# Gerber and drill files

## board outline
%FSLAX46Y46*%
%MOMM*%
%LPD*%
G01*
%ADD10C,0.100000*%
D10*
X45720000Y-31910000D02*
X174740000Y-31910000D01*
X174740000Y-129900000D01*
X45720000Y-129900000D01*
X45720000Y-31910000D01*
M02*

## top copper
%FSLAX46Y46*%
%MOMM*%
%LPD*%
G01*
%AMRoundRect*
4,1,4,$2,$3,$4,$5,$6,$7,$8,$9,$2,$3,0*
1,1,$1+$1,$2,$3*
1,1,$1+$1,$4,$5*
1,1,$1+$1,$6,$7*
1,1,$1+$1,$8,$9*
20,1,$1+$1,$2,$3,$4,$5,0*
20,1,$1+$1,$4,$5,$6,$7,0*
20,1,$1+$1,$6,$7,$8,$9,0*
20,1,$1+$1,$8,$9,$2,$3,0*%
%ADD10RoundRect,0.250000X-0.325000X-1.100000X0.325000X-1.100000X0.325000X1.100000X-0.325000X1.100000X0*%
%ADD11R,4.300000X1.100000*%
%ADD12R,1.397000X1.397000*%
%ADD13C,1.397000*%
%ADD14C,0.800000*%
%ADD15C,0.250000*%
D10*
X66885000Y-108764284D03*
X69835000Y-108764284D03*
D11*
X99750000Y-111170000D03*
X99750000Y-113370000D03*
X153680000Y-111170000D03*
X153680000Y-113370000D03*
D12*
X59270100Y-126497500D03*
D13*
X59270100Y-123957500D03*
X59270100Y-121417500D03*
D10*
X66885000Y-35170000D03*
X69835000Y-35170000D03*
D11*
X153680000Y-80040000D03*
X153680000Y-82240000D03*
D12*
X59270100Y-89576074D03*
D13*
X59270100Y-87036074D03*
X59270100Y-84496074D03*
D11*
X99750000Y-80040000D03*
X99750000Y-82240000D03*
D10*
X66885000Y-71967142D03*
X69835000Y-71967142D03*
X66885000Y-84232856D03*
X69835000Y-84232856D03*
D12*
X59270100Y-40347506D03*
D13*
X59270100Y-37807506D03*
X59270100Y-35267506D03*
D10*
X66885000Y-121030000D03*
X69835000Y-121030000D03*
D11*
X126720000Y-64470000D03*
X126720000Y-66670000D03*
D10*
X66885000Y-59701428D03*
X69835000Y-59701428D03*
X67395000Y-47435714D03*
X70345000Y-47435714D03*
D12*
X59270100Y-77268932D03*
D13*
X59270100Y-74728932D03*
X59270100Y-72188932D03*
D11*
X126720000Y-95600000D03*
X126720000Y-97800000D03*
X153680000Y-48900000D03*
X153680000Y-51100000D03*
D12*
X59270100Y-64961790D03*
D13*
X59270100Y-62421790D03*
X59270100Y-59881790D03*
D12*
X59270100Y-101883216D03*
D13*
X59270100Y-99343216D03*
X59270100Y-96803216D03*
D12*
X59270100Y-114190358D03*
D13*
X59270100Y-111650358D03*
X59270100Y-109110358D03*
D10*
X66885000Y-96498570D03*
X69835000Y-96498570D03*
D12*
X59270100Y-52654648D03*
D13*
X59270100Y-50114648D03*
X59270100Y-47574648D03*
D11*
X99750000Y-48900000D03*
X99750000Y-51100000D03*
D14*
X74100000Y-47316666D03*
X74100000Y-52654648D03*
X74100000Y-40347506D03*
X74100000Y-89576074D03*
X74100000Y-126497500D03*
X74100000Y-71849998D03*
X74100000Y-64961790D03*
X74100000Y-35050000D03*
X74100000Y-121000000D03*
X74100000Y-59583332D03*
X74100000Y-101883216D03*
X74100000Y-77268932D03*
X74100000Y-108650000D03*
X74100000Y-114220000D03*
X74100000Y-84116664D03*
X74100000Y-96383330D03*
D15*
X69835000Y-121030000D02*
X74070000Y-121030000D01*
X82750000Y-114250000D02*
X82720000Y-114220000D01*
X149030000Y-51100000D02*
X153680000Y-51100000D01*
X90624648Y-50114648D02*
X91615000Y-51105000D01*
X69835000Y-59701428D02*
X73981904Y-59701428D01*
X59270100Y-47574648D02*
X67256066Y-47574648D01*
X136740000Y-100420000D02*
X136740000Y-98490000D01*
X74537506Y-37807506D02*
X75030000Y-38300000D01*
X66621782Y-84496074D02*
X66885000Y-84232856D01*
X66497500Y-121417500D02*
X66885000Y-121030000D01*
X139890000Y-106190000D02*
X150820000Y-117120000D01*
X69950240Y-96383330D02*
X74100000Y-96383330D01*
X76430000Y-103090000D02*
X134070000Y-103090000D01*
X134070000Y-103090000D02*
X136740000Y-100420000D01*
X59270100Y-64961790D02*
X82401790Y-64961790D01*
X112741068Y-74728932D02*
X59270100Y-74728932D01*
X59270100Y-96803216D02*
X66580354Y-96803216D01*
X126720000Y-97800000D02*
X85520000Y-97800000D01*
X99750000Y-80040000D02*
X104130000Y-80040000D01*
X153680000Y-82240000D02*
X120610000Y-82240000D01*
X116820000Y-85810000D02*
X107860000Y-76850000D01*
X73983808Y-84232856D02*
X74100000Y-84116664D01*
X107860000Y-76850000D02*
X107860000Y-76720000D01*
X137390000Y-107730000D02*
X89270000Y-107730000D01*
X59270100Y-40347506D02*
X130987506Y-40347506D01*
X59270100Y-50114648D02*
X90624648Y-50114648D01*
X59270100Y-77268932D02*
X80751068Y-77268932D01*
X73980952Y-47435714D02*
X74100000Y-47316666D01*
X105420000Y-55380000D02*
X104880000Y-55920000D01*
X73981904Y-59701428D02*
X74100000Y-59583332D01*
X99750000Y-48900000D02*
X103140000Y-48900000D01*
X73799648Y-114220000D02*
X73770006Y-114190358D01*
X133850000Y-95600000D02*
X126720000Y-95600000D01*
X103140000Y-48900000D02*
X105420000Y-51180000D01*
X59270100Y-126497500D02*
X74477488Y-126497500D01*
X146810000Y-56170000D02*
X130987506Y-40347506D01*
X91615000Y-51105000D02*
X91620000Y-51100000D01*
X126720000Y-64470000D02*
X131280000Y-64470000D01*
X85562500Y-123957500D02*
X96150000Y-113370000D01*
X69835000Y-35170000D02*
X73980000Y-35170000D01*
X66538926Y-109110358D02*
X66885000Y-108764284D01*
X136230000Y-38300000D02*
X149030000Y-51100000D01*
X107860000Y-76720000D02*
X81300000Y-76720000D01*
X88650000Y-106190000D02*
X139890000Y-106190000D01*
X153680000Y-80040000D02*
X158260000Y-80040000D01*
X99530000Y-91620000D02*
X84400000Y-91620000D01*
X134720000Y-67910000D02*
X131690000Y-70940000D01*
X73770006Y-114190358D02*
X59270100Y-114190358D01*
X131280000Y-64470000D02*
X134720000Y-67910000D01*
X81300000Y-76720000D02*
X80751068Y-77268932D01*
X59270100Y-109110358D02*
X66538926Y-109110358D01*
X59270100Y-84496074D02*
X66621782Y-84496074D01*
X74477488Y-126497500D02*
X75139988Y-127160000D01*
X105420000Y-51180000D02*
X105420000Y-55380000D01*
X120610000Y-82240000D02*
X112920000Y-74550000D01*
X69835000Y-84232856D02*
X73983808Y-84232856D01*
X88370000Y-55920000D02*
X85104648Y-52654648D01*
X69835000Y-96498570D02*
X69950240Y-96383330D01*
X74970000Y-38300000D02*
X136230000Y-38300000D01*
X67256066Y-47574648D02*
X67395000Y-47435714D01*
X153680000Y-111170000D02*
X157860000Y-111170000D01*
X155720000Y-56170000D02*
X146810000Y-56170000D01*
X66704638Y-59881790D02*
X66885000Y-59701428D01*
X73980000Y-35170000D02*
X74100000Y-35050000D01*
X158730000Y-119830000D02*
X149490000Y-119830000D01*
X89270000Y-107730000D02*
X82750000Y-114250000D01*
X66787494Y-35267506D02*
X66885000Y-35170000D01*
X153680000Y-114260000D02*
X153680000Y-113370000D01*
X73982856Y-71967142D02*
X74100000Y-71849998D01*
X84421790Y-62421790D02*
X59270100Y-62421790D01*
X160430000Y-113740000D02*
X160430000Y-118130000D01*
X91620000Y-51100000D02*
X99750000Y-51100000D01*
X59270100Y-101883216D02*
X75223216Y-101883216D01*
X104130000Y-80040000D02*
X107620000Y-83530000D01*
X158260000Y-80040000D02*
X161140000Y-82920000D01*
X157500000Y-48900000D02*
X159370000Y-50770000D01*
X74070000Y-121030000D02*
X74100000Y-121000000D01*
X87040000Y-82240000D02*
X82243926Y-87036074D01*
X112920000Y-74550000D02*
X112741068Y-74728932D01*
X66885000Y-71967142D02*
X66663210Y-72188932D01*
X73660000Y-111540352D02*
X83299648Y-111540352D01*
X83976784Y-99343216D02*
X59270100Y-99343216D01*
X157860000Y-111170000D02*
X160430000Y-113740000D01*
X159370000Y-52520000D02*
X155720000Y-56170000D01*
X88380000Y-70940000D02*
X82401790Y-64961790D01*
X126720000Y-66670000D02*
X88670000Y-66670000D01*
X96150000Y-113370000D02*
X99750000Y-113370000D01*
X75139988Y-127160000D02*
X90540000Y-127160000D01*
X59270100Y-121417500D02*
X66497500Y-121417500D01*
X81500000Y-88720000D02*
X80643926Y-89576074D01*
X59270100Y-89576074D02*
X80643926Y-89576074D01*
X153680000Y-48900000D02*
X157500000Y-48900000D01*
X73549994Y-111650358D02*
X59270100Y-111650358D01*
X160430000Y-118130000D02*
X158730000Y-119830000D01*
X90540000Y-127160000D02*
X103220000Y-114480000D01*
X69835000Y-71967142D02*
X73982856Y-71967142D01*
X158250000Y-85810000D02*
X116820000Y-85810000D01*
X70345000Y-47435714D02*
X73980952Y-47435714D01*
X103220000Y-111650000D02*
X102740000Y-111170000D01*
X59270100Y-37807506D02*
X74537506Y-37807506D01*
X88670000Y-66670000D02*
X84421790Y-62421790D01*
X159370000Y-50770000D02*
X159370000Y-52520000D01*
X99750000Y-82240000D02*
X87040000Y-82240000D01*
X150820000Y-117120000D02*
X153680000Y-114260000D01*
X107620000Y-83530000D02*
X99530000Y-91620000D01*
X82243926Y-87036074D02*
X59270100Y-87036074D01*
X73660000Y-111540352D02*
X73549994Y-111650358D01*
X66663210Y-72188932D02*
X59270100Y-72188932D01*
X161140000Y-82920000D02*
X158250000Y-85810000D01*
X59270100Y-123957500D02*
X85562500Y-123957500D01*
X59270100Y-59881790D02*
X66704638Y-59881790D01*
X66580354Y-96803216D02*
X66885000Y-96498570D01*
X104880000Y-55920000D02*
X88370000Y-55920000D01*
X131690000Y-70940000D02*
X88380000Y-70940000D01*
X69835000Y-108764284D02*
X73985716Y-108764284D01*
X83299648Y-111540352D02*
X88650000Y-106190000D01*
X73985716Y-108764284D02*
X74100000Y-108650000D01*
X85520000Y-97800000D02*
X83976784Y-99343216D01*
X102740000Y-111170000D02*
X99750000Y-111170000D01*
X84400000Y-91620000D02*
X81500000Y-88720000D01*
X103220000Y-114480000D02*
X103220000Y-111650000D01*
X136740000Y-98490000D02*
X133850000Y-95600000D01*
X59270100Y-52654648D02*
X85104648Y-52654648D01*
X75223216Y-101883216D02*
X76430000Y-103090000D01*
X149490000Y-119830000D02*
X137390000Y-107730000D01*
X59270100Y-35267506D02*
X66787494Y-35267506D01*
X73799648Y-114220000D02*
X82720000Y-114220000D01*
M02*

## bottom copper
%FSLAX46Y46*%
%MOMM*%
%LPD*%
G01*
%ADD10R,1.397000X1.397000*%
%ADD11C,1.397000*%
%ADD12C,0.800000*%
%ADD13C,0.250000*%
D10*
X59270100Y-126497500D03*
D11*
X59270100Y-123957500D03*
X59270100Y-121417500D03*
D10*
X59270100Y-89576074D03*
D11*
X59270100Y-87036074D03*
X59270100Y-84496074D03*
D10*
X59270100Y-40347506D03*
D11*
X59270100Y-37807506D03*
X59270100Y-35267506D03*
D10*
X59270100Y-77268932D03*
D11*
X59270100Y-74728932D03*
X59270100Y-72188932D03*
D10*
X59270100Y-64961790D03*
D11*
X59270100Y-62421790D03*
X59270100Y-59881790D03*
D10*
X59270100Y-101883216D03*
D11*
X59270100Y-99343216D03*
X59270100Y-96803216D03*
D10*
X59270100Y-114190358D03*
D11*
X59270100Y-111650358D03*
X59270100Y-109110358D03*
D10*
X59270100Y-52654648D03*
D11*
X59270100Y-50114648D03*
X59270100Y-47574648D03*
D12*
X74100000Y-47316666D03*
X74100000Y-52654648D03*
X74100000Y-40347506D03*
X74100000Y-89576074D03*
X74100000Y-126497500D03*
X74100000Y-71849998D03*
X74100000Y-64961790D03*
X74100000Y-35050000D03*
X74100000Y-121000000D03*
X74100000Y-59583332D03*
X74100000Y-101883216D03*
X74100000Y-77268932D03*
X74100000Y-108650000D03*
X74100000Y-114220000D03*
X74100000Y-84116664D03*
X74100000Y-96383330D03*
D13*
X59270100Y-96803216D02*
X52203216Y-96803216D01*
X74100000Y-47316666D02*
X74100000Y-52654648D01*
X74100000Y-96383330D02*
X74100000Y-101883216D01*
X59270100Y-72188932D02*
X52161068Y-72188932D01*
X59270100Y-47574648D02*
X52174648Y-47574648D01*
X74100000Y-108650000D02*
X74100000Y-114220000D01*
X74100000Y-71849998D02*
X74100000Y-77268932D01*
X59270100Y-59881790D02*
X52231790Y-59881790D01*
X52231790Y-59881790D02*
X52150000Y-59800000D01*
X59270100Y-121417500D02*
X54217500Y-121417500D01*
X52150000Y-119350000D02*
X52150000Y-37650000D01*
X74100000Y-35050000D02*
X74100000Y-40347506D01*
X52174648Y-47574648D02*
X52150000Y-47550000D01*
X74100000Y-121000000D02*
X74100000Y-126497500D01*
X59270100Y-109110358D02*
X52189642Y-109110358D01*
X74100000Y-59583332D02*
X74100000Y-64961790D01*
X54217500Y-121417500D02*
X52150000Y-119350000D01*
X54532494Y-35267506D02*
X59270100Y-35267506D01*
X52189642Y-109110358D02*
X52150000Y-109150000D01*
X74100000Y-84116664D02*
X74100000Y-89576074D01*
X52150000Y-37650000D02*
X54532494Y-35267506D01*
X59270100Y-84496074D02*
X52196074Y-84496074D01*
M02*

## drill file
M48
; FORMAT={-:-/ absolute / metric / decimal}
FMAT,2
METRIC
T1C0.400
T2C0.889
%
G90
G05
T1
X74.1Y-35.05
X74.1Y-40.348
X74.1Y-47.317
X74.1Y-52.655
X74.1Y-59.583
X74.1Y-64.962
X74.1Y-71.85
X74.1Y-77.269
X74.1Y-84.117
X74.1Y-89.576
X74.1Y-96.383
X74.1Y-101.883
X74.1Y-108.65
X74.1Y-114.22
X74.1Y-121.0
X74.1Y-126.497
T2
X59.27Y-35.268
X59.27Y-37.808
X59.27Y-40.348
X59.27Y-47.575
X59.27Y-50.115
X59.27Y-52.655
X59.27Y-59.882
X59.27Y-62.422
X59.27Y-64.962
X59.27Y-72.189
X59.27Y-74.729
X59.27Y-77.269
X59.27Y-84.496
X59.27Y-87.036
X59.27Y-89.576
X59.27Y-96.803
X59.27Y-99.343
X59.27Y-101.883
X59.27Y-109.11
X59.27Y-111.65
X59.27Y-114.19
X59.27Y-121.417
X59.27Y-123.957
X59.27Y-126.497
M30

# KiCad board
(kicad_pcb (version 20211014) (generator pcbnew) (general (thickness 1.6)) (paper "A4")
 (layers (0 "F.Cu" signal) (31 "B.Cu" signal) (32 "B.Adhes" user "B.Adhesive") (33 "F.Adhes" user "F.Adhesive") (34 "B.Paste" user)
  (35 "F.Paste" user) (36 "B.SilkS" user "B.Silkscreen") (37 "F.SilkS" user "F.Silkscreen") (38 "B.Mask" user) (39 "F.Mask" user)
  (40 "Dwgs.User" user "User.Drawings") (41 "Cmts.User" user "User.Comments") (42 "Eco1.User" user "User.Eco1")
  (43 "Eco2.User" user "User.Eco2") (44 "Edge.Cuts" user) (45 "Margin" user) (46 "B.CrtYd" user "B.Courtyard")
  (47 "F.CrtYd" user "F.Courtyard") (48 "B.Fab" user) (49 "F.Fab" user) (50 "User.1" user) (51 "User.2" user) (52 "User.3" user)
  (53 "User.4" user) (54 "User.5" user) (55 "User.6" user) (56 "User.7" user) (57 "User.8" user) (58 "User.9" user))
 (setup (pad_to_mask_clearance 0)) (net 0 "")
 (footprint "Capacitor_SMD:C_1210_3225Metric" (layer "F.Cu") (at 68.36 108.764284)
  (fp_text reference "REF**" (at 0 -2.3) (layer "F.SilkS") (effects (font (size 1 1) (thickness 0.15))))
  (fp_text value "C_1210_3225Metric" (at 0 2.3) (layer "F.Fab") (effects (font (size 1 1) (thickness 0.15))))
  (pad "1" smd roundrect (at -1.475 0) (size 1.15 2.7) (layers "F.Cu" "F.Paste" "F.Mask") (roundrect_rratio 0.2173913043))
  (pad "2" smd roundrect (at 1.475 0) (size 1.15 2.7) (layers "F.Cu" "F.Paste" "F.Mask") (roundrect_rratio 0.2173913043)))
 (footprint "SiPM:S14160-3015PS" (layer "F.Cu") (at 100 112.27)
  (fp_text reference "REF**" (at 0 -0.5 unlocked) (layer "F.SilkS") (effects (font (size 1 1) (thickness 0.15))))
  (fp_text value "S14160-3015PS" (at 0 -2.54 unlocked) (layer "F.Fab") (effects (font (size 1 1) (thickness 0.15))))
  (pad "1" smd rect (at -0.25 -1.1) (size 4.3 1.1) (layers "F.Cu" "F.Paste" "F.Mask"))
  (pad "2" smd rect (at -0.25 1.1) (size 4.3 1.1) (layers "F.Cu" "F.Paste" "F.Mask")))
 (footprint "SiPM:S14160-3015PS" (layer "F.Cu") (at 153.93 112.27)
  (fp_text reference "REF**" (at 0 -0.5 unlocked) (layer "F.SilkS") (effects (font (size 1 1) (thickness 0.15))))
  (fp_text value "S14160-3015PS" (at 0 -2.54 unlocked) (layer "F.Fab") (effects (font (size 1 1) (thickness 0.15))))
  (pad "1" smd rect (at -0.25 -1.1) (size 4.3 1.1) (layers "F.Cu" "F.Paste" "F.Mask"))
  (pad "2" smd rect (at -0.25 1.1) (size 4.3 1.1) (layers "F.Cu" "F.Paste" "F.Mask")))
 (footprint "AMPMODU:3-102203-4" (layer "F.Cu") (at 59.2701 126.4975 90)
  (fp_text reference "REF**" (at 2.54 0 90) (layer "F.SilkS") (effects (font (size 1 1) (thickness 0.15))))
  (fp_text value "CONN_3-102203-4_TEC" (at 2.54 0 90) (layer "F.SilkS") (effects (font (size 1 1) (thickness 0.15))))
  (pad "1" thru_hole rect locked (at 0 0 90) (size 1.397 1.397) (drill 0.889) (layers *.Cu *.Mask))
  (pad "2" thru_hole circle locked (at 2.54 0 90) (size 1.397 1.397) (drill 0.889) (layers *.Cu *.Mask))
  (pad "3" thru_hole circle locked (at 5.08 0 90) (size 1.397 1.397) (drill 0.889) (layers *.Cu *.Mask)))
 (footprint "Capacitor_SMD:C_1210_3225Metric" (layer "F.Cu") (at 68.36 35.17)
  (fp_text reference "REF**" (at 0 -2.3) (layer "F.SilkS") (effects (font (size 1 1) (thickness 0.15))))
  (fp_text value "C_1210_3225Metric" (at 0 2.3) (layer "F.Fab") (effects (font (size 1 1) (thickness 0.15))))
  (pad "1" smd roundrect (at -1.475 0) (size 1.15 2.7) (layers "F.Cu" "F.Paste" "F.Mask") (roundrect_rratio 0.2173913043))
  (pad "2" smd roundrect (at 1.475 0) (size 1.15 2.7) (layers "F.Cu" "F.Paste" "F.Mask") (roundrect_rratio 0.2173913043)))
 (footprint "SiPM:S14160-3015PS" (layer "F.Cu") (at 153.93 81.14)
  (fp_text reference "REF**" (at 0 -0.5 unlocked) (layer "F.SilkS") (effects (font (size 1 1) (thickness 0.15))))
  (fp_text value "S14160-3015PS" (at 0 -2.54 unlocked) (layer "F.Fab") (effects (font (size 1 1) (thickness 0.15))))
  (pad "1" smd rect (at -0.25 -1.1) (size 4.3 1.1) (layers "F.Cu" "F.Paste" "F.Mask"))
  (pad "2" smd rect (at -0.25 1.1) (size 4.3 1.1) (layers "F.Cu" "F.Paste" "F.Mask")))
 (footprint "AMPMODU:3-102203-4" (layer "F.Cu") (at 59.2701 89.576074 90)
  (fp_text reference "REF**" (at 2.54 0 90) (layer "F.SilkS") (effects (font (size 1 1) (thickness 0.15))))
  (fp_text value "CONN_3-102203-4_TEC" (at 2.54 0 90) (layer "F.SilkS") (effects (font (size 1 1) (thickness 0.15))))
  (pad "1" thru_hole rect locked (at 0 0 90) (size 1.397 1.397) (drill 0.889) (layers *.Cu *.Mask))
  (pad "2" thru_hole circle locked (at 2.54 0 90) (size 1.397 1.397) (drill 0.889) (layers *.Cu *.Mask))
  (pad "3" thru_hole circle locked (at 5.08 0 90) (size 1.397 1.397) (drill 0.889) (layers *.Cu *.Mask)))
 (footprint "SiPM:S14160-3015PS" (layer "F.Cu") (at 100 81.14)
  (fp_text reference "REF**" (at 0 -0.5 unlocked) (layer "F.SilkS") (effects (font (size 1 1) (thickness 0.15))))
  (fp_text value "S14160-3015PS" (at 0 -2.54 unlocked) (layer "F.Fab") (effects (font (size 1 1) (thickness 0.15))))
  (pad "1" smd rect (at -0.25 -1.1) (size 4.3 1.1) (layers "F.Cu" "F.Paste" "F.Mask"))
  (pad "2" smd rect (at -0.25 1.1) (size 4.3 1.1) (layers "F.Cu" "F.Paste" "F.Mask")))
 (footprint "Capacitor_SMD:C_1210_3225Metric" (layer "F.Cu") (at 68.36 71.967142)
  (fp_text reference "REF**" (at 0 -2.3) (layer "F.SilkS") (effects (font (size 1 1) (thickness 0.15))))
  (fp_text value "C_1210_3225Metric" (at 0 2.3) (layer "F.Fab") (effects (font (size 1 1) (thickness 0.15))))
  (pad "1" smd roundrect (at -1.475 0) (size 1.15 2.7) (layers "F.Cu" "F.Paste" "F.Mask") (roundrect_rratio 0.2173913043))
  (pad "2" smd roundrect (at 1.475 0) (size 1.15 2.7) (layers "F.Cu" "F.Paste" "F.Mask") (roundrect_rratio 0.2173913043)))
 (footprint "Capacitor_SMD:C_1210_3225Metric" (layer "F.Cu") (at 68.36 84.232856)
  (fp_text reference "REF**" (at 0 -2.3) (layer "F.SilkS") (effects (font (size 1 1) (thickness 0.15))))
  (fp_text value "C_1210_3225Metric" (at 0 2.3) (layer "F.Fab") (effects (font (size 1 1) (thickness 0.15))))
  (pad "1" smd roundrect (at -1.475 0) (size 1.15 2.7) (layers "F.Cu" "F.Paste" "F.Mask") (roundrect_rratio 0.2173913043))
  (pad "2" smd roundrect (at 1.475 0) (size 1.15 2.7) (layers "F.Cu" "F.Paste" "F.Mask") (roundrect_rratio 0.2173913043)))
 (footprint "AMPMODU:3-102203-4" (layer "F.Cu") (at 59.2701 40.347506 90)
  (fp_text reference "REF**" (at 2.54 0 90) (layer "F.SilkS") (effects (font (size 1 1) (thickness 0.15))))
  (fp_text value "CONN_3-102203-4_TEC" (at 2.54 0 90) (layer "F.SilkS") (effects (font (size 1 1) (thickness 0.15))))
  (pad "1" thru_hole rect locked (at 0 0 90) (size 1.397 1.397) (drill 0.889) (layers *.Cu *.Mask))
  (pad "2" thru_hole circle locked (at 2.54 0 90) (size 1.397 1.397) (drill 0.889) (layers *.Cu *.Mask))
  (pad "3" thru_hole circle locked (at 5.08 0 90) (size 1.397 1.397) (drill 0.889) (layers *.Cu *.Mask)))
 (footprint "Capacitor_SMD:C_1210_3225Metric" (layer "F.Cu") (at 68.36 121.03)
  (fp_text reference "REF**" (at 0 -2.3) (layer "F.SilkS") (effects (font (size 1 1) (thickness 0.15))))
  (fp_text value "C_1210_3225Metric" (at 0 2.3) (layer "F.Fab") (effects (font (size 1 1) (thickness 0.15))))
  (pad "1" smd roundrect (at -1.475 0) (size 1.15 2.7) (layers "F.Cu" "F.Paste" "F.Mask") (roundrect_rratio 0.2173913043))
  (pad "2" smd roundrect (at 1.475 0) (size 1.15 2.7) (layers "F.Cu" "F.Paste" "F.Mask") (roundrect_rratio 0.2173913043)))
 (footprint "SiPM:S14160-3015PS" (layer "F.Cu") (at 126.97 65.57)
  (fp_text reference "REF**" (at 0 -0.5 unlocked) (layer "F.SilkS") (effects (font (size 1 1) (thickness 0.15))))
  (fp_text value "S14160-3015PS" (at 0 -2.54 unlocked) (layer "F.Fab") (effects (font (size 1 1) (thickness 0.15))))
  (pad "1" smd rect (at -0.25 -1.1) (size 4.3 1.1) (layers "F.Cu" "F.Paste" "F.Mask"))
  (pad "2" smd rect (at -0.25 1.1) (size 4.3 1.1) (layers "F.Cu" "F.Paste" "F.Mask")))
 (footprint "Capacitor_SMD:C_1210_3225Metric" (layer "F.Cu") (at 68.36 59.701428)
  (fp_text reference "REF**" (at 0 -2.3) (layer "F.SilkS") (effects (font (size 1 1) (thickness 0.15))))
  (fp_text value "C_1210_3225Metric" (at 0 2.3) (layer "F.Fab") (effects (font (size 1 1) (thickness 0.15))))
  (pad "1" smd roundrect (at -1.475 0) (size 1.15 2.7) (layers "F.Cu" "F.Paste" "F.Mask") (roundrect_rratio 0.2173913043))
  (pad "2" smd roundrect (at 1.475 0) (size 1.15 2.7) (layers "F.Cu" "F.Paste" "F.Mask") (roundrect_rratio 0.2173913043)))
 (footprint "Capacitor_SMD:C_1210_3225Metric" (layer "F.Cu") (at 68.87 47.435714)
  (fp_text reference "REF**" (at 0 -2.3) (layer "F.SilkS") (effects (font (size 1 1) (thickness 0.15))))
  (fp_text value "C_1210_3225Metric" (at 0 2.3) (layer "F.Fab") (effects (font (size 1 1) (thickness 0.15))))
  (pad "1" smd roundrect (at -1.475 0) (size 1.15 2.7) (layers "F.Cu" "F.Paste" "F.Mask") (roundrect_rratio 0.2173913043))
  (pad "2" smd roundrect (at 1.475 0) (size 1.15 2.7) (layers "F.Cu" "F.Paste" "F.Mask") (roundrect_rratio 0.2173913043)))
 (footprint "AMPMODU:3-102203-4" (layer "F.Cu") (at 59.2701 77.268932 90)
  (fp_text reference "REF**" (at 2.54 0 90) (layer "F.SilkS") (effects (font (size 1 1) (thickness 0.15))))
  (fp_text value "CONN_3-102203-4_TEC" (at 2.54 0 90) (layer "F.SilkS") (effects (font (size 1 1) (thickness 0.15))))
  (pad "1" thru_hole rect locked (at 0 0 90) (size 1.397 1.397) (drill 0.889) (layers *.Cu *.Mask))
  (pad "2" thru_hole circle locked (at 2.54 0 90) (size 1.397 1.397) (drill 0.889) (layers *.Cu *.Mask))
  (pad "3" thru_hole circle locked (at 5.08 0 90) (size 1.397 1.397) (drill 0.889) (layers *.Cu *.Mask)))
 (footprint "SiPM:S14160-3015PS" (layer "F.Cu") (at 126.97 96.7)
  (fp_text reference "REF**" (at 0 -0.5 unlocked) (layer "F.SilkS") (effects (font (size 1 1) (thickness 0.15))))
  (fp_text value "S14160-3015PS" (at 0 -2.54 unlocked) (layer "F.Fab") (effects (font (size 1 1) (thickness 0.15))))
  (pad "1" smd rect (at -0.25 -1.1) (size 4.3 1.1) (layers "F.Cu" "F.Paste" "F.Mask"))
  (pad "2" smd rect (at -0.25 1.1) (size 4.3 1.1) (layers "F.Cu" "F.Paste" "F.Mask")))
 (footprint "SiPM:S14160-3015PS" (layer "F.Cu") (at 153.93 50)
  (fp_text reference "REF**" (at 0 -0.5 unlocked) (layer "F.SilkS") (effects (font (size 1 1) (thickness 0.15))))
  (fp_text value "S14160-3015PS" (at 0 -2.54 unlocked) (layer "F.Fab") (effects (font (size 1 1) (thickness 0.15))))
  (pad "1" smd rect (at -0.25 -1.1) (size 4.3 1.1) (layers "F.Cu" "F.Paste" "F.Mask"))
  (pad "2" smd rect (at -0.25 1.1) (size 4.3 1.1) (layers "F.Cu" "F.Paste" "F.Mask")))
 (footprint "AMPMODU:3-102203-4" (layer "F.Cu") (at 59.2701 64.96179 90)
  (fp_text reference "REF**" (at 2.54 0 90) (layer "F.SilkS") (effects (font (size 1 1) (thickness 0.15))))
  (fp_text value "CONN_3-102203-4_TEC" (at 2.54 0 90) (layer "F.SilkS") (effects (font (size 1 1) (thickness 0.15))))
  (pad "1" thru_hole rect locked (at 0 0 90) (size 1.397 1.397) (drill 0.889) (layers *.Cu *.Mask))
  (pad "2" thru_hole circle locked (at 2.54 0 90) (size 1.397 1.397) (drill 0.889) (layers *.Cu *.Mask))
  (pad "3" thru_hole circle locked (at 5.08 0 90) (size 1.397 1.397) (drill 0.889) (layers *.Cu *.Mask)))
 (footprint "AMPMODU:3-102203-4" (layer "F.Cu") (at 59.2701 101.883216 90)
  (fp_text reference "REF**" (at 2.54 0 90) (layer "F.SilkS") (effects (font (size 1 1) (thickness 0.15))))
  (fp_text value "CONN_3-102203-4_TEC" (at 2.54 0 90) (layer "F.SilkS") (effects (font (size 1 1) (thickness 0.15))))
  (pad "1" thru_hole rect locked (at 0 0 90) (size 1.397 1.397) (drill 0.889) (layers *.Cu *.Mask))
  (pad "2" thru_hole circle locked (at 2.54 0 90) (size 1.397 1.397) (drill 0.889) (layers *.Cu *.Mask))
  (pad "3" thru_hole circle locked (at 5.08 0 90) (size 1.397 1.397) (drill 0.889) (layers *.Cu *.Mask)))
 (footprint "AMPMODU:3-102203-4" (layer "F.Cu") (at 59.2701 114.190358 90)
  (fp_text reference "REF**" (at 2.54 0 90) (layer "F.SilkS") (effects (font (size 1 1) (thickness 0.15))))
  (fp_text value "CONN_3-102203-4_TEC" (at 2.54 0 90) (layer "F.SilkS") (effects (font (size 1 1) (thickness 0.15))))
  (pad "1" thru_hole rect locked (at 0 0 90) (size 1.397 1.397) (drill 0.889) (layers *.Cu *.Mask))
  (pad "2" thru_hole circle locked (at 2.54 0 90) (size 1.397 1.397) (drill 0.889) (layers *.Cu *.Mask))
  (pad "3" thru_hole circle locked (at 5.08 0 90) (size 1.397 1.397) (drill 0.889) (layers *.Cu *.Mask)))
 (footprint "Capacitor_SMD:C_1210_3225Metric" (layer "F.Cu") (at 68.36 96.49857)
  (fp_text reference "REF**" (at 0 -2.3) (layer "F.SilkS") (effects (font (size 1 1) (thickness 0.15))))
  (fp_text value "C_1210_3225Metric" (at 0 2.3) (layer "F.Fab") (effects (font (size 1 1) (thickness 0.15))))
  (pad "1" smd roundrect (at -1.475 0) (size 1.15 2.7) (layers "F.Cu" "F.Paste" "F.Mask") (roundrect_rratio 0.2173913043))
  (pad "2" smd roundrect (at 1.475 0) (size 1.15 2.7) (layers "F.Cu" "F.Paste" "F.Mask") (roundrect_rratio 0.2173913043)))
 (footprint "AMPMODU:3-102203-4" (layer "F.Cu") (at 59.2701 52.654648 90)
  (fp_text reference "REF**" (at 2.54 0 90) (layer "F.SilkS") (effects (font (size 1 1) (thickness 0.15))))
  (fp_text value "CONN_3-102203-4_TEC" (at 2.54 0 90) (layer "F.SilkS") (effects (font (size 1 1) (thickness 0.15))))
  (pad "1" thru_hole rect locked (at 0 0 90) (size 1.397 1.397) (drill 0.889) (layers *.Cu *.Mask))
  (pad "2" thru_hole circle locked (at 2.54 0 90) (size 1.397 1.397) (drill 0.889) (layers *.Cu *.Mask))
  (pad "3" thru_hole circle locked (at 5.08 0 90) (size 1.397 1.397) (drill 0.889) (layers *.Cu *.Mask)))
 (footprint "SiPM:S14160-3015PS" (layer "F.Cu") (at 100 50)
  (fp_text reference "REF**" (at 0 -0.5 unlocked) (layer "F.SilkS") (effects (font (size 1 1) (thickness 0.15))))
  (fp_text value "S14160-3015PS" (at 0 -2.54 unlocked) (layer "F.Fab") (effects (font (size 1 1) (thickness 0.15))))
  (pad "1" smd rect (at -0.25 -1.1) (size 4.3 1.1) (layers "F.Cu" "F.Paste" "F.Mask"))
  (pad "2" smd rect (at -0.25 1.1) (size 4.3 1.1) (layers "F.Cu" "F.Paste" "F.Mask")))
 (gr_rect (start 45.72 31.91) (end 174.74 129.9) (layer "Edge.Cuts") (width 0.1) (fill none))
 (segment (start 69.835 121.03) (end 74.07 121.03) (width 0.25) (layer "F.Cu") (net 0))
 (segment (start 82.75 114.25) (end 82.72 114.22) (width 0.25) (layer "F.Cu") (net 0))
 (segment (start 149.03 51.1) (end 153.68 51.1) (width 0.25) (layer "F.Cu") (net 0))
 (segment (start 90.624648 50.114648) (end 91.615 51.105) (width 0.25) (layer "F.Cu") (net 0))
 (segment (start 69.835 59.701428) (end 73.981904 59.701428) (width 0.25) (layer "F.Cu") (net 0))
 (segment (start 59.2701 47.574648) (end 67.256066 47.574648) (width 0.25) (layer "F.Cu") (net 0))
 (segment (start 136.74 100.42) (end 136.74 98.49) (width 0.25) (layer "F.Cu") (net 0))
 (segment (start 74.537506 37.807506) (end 75.03 38.3) (width 0.25) (layer "F.Cu") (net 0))
 (segment (start 66.621782 84.496074) (end 66.885 84.232856) (width 0.25) (layer "F.Cu") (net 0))
 (segment (start 66.4975 121.4175) (end 66.885 121.03) (width 0.25) (layer "F.Cu") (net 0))
 (segment (start 139.89 106.19) (end 150.82 117.12) (width 0.25) (layer "F.Cu") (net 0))
 (segment (start 69.95024 96.38333) (end 74.1 96.38333) (width 0.25) (layer "F.Cu") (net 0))
 (segment (start 76.43 103.09) (end 134.07 103.09) (width 0.25) (layer "F.Cu") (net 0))
 (segment (start 134.07 103.09) (end 136.74 100.42) (width 0.25) (layer "F.Cu") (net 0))
 (segment (start 59.2701 64.96179) (end 82.40179 64.96179) (width 0.25) (layer "F.Cu") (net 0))
 (segment (start 112.741068 74.728932) (end 59.2701 74.728932) (width 0.25) (layer "F.Cu") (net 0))
 (segment (start 59.2701 96.803216) (end 66.580354 96.803216) (width 0.25) (layer "F.Cu") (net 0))
 (segment (start 126.72 97.8) (end 85.52 97.8) (width 0.25) (layer "F.Cu") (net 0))
 (segment (start 99.75 80.04) (end 104.13 80.04) (width 0.25) (layer "F.Cu") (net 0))
 (segment (start 153.68 82.24) (end 120.61 82.24) (width 0.25) (layer "F.Cu") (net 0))
 (segment (start 116.82 85.81) (end 107.86 76.85) (width 0.25) (layer "F.Cu") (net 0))
 (segment (start 73.983808 84.232856) (end 74.1 84.116664) (width 0.25) (layer "F.Cu") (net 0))
 (segment (start 107.86 76.85) (end 107.86 76.72) (width 0.25) (layer "F.Cu") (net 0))
 (segment (start 137.39 107.73) (end 89.27 107.73) (width 0.25) (layer "F.Cu") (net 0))
 (segment (start 59.2701 40.347506) (end 130.987506 40.347506) (width 0.25) (layer "F.Cu") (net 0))
 (segment (start 59.2701 50.114648) (end 90.624648 50.114648) (width 0.25) (layer "F.Cu") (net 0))
 (segment (start 59.2701 77.268932) (end 80.751068 77.268932) (width 0.25) (layer "F.Cu") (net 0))
 (segment (start 73.980952 47.435714) (end 74.1 47.316666) (width 0.25) (layer "F.Cu") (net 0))
 (segment (start 105.42 55.38) (end 104.88 55.92) (width 0.25) (layer "F.Cu") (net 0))
 (segment (start 73.981904 59.701428) (end 74.1 59.583332) (width 0.25) (layer "F.Cu") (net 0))
 (segment (start 99.75 48.9) (end 103.14 48.9) (width 0.25) (layer "F.Cu") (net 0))
 (segment (start 73.799648 114.22) (end 73.770006 114.190358) (width 0.25) (layer "F.Cu") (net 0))
 (segment (start 133.85 95.6) (end 126.72 95.6) (width 0.25) (layer "F.Cu") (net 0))
 (segment (start 103.14 48.9) (end 105.42 51.18) (width 0.25) (layer "F.Cu") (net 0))
 (segment (start 59.2701 126.4975) (end 74.477488 126.4975) (width 0.25) (layer "F.Cu") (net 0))
 (segment (start 146.81 56.17) (end 130.987506 40.347506) (width 0.25) (layer "F.Cu") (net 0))
 (segment (start 91.615 51.105) (end 91.62 51.1) (width 0.25) (layer "F.Cu") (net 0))
 (segment (start 126.72 64.47) (end 131.28 64.47) (width 0.25) (layer "F.Cu") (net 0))
 (segment (start 85.5625 123.9575) (end 96.15 113.37) (width 0.25) (layer "F.Cu") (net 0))
 (segment (start 69.835 35.17) (end 73.98 35.17) (width 0.25) (layer "F.Cu") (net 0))
 (segment (start 66.538926 109.110358) (end 66.885 108.764284) (width 0.25) (layer "F.Cu") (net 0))
 (segment (start 136.23 38.3) (end 149.03 51.1) (width 0.25) (layer "F.Cu") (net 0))
 (segment (start 107.86 76.72) (end 81.3 76.72) (width 0.25) (layer "F.Cu") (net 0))
 (segment (start 88.65 106.19) (end 139.89 106.19) (width 0.25) (layer "F.Cu") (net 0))
 (segment (start 153.68 80.04) (end 158.26 80.04) (width 0.25) (layer "F.Cu") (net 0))
 (segment (start 99.53 91.62) (end 84.4 91.62) (width 0.25) (layer "F.Cu") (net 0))
 (segment (start 134.72 67.91) (end 131.69 70.94) (width 0.25) (layer "F.Cu") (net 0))
 (segment (start 73.770006 114.190358) (end 59.2701 114.190358) (width 0.25) (layer "F.Cu") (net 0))
 (segment (start 131.28 64.47) (end 134.72 67.91) (width 0.25) (layer "F.Cu") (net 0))
 (segment (start 81.3 76.72) (end 80.751068 77.268932) (width 0.25) (layer "F.Cu") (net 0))
 (segment (start 59.2701 109.110358) (end 66.538926 109.110358) (width 0.25) (layer "F.Cu") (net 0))
 (segment (start 59.2701 84.496074) (end 66.621782 84.496074) (width 0.25) (layer "F.Cu") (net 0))
 (segment (start 74.477488 126.4975) (end 75.139988 127.16) (width 0.25) (layer "F.Cu") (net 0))
 (segment (start 105.42 51.18) (end 105.42 55.38) (width 0.25) (layer "F.Cu") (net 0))
 (segment (start 120.61 82.24) (end 112.92 74.55) (width 0.25) (layer "F.Cu") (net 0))
 (segment (start 69.835 84.232856) (end 73.983808 84.232856) (width 0.25) (layer "F.Cu") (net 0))
 (segment (start 88.37 55.92) (end 85.104648 52.654648) (width 0.25) (layer "F.Cu") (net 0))
 (segment (start 69.835 96.49857) (end 69.95024 96.38333) (width 0.25) (layer "F.Cu") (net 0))
 (segment (start 74.97 38.3) (end 136.23 38.3) (width 0.25) (layer "F.Cu") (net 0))
 (segment (start 67.256066 47.574648) (end 67.395 47.435714) (width 0.25) (layer "F.Cu") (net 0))
 (segment (start 153.68 111.17) (end 157.86 111.17) (width 0.25) (layer "F.Cu") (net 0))
 (segment (start 155.72 56.17) (end 146.81 56.17) (width 0.25) (layer "F.Cu") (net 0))
 (segment (start 66.704638 59.88179) (end 66.885 59.701428) (width 0.25) (layer "F.Cu") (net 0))
 (segment (start 73.98 35.17) (end 74.1 35.05) (width 0.25) (layer "F.Cu") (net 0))
 (segment (start 158.73 119.83) (end 149.49 119.83) (width 0.25) (layer "F.Cu") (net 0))
 (segment (start 89.27 107.73) (end 82.75 114.25) (width 0.25) (layer "F.Cu") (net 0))
 (segment (start 66.787494 35.267506) (end 66.885 35.17) (width 0.25) (layer "F.Cu") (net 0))
 (segment (start 153.68 114.26) (end 153.68 113.37) (width 0.25) (layer "F.Cu") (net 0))
 (segment (start 73.982856 71.967142) (end 74.1 71.849998) (width 0.25) (layer "F.Cu") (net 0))
 (segment (start 84.42179 62.42179) (end 59.2701 62.42179) (width 0.25) (layer "F.Cu") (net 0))
 (segment (start 160.43 113.74) (end 160.43 118.13) (width 0.25) (layer "F.Cu") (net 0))
 (segment (start 91.62 51.1) (end 99.75 51.1) (width 0.25) (layer "F.Cu") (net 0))
 (segment (start 59.2701 101.883216) (end 75.223216 101.883216) (width 0.25) (layer "F.Cu") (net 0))
 (segment (start 104.13 80.04) (end 107.62 83.53) (width 0.25) (layer "F.Cu") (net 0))
 (segment (start 158.26 80.04) (end 161.14 82.92) (width 0.25) (layer "F.Cu") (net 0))
 (segment (start 157.5 48.9) (end 159.37 50.77) (width 0.25) (layer "F.Cu") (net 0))
 (segment (start 74.07 121.03) (end 74.1 121) (width 0.25) (layer "F.Cu") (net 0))
 (segment (start 87.04 82.24) (end 82.243926 87.036074) (width 0.25) (layer "F.Cu") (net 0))
 (segment (start 112.92 74.55) (end 112.741068 74.728932) (width 0.25) (layer "F.Cu") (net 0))
 (segment (start 66.885 71.967142) (end 66.66321 72.188932) (width 0.25) (layer "F.Cu") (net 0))
 (segment (start 73.66 111.540352) (end 83.299648 111.540352) (width 0.25) (layer "F.Cu") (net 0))
 (segment (start 83.976784 99.343216) (end 59.2701 99.343216) (width 0.25) (layer "F.Cu") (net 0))
 (segment (start 157.86 111.17) (end 160.43 113.74) (width 0.25) (layer "F.Cu") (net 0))
 (segment (start 159.37 52.52) (end 155.72 56.17) (width 0.25) (layer "F.Cu") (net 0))
 (segment (start 88.38 70.94) (end 82.40179 64.96179) (width 0.25) (layer "F.Cu") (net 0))
 (segment (start 126.72 66.67) (end 88.67 66.67) (width 0.25) (layer "F.Cu") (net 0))
 (segment (start 96.15 113.37) (end 99.75 113.37) (width 0.25) (layer "F.Cu") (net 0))
 (segment (start 75.139988 127.16) (end 90.54 127.16) (width 0.25) (layer "F.Cu") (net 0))
 (segment (start 59.2701 121.4175) (end 66.4975 121.4175) (width 0.25) (layer "F.Cu") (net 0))
 (segment (start 81.5 88.72) (end 80.643926 89.576074) (width 0.25) (layer "F.Cu") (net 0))
 (segment (start 59.2701 89.576074) (end 80.643926 89.576074) (width 0.25) (layer "F.Cu") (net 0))
 (segment (start 153.68 48.9) (end 157.5 48.9) (width 0.25) (layer "F.Cu") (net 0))
 (segment (start 73.549994 111.650358) (end 59.2701 111.650358) (width 0.25) (layer "F.Cu") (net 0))
 (segment (start 160.43 118.13) (end 158.73 119.83) (width 0.25) (layer "F.Cu") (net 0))
 (segment (start 90.54 127.16) (end 103.22 114.48) (width 0.25) (layer "F.Cu") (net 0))
 (segment (start 69.835 71.967142) (end 73.982856 71.967142) (width 0.25) (layer "F.Cu") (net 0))
 (segment (start 158.25 85.81) (end 116.82 85.81) (width 0.25) (layer "F.Cu") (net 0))
 (segment (start 70.345 47.435714) (end 73.980952 47.435714) (width 0.25) (layer "F.Cu") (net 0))
 (segment (start 103.22 111.65) (end 102.74 111.17) (width 0.25) (layer "F.Cu") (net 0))
 (segment (start 59.2701 37.807506) (end 74.537506 37.807506) (width 0.25) (layer "F.Cu") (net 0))
 (segment (start 88.67 66.67) (end 84.42179 62.42179) (width 0.25) (layer "F.Cu") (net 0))
 (segment (start 159.37 50.77) (end 159.37 52.52) (width 0.25) (layer "F.Cu") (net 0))
 (segment (start 99.75 82.24) (end 87.04 82.24) (width 0.25) (layer "F.Cu") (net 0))
 (segment (start 150.82 117.12) (end 153.68 114.26) (width 0.25) (layer "F.Cu") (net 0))
 (segment (start 107.62 83.53) (end 99.53 91.62) (width 0.25) (layer "F.Cu") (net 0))
 (segment (start 82.243926 87.036074) (end 59.2701 87.036074) (width 0.25) (layer "F.Cu") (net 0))
 (segment (start 73.66 111.540352) (end 73.549994 111.650358) (width 0.25) (layer "F.Cu") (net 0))
 (segment (start 66.66321 72.188932) (end 59.2701 72.188932) (width 0.25) (layer "F.Cu") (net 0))
 (segment (start 161.14 82.92) (end 158.25 85.81) (width 0.25) (layer "F.Cu") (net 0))
 (segment (start 59.2701 123.9575) (end 85.5625 123.9575) (width 0.25) (layer "F.Cu") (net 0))
 (segment (start 59.2701 59.88179) (end 66.704638 59.88179) (width 0.25) (layer "F.Cu") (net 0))
 (segment (start 66.580354 96.803216) (end 66.885 96.49857) (width 0.25) (layer "F.Cu") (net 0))
 (segment (start 104.88 55.92) (end 88.37 55.92) (width 0.25) (layer "F.Cu") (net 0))
 (segment (start 131.69 70.94) (end 88.38 70.94) (width 0.25) (layer "F.Cu") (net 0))
 (segment (start 69.835 108.764284) (end 73.985716 108.764284) (width 0.25) (layer "F.Cu") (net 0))
 (segment (start 83.299648 111.540352) (end 88.65 106.19) (width 0.25) (layer "F.Cu") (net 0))
 (segment (start 73.985716 108.764284) (end 74.1 108.65) (width 0.25) (layer "F.Cu") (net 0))
 (segment (start 85.52 97.8) (end 83.976784 99.343216) (width 0.25) (layer "F.Cu") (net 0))
 (segment (start 102.74 111.17) (end 99.75 111.17) (width 0.25) (layer "F.Cu") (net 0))
 (segment (start 84.4 91.62) (end 81.5 88.72) (width 0.25) (layer "F.Cu") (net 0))
 (segment (start 103.22 114.48) (end 103.22 111.65) (width 0.25) (layer "F.Cu") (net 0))
 (segment (start 136.74 98.49) (end 133.85 95.6) (width 0.25) (layer "F.Cu") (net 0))
 (segment (start 59.2701 52.654648) (end 85.104648 52.654648) (width 0.25) (layer "F.Cu") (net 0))
 (segment (start 75.223216 101.883216) (end 76.43 103.09) (width 0.25) (layer "F.Cu") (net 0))
 (segment (start 149.49 119.83) (end 137.39 107.73) (width 0.25) (layer "F.Cu") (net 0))
 (segment (start 59.2701 35.267506) (end 66.787494 35.267506) (width 0.25) (layer "F.Cu") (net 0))
 (segment (start 73.799648 114.22) (end 82.72 114.22) (width 0.25) (layer "F.Cu") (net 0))
 (via (at 74.1 47.316666) (size 0.8) (drill 0.4) (layers "F.Cu" "B.Cu") (free) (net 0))
 (via (at 74.1 52.654648) (size 0.8) (drill 0.4) (layers "F.Cu" "B.Cu") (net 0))
 (via (at 74.1 40.347506) (size 0.8) (drill 0.4) (layers "F.Cu" "B.Cu") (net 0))
 (via (at 74.1 89.576074) (size 0.8) (drill 0.4) (layers "F.Cu" "B.Cu") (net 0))
 (via (at 74.1 126.4975) (size 0.8) (drill 0.4) (layers "F.Cu" "B.Cu") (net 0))
 (via (at 74.1 71.849998) (size 0.8) (drill 0.4) (layers "F.Cu" "B.Cu") (free) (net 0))
 (via (at 74.1 64.96179) (size 0.8) (drill 0.4) (layers "F.Cu" "B.Cu") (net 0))
 (via (at 74.1 35.05) (size 0.8) (drill 0.4) (layers "F.Cu" "B.Cu") (free) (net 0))
 (via (at 74.1 121) (size 0.8) (drill 0.4) (layers "F.Cu" "B.Cu") (free) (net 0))
 (via (at 74.1 59.583332) (size 0.8) (drill 0.4) (layers "F.Cu" "B.Cu") (free) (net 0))
 (via (at 74.1 101.883216) (size 0.8) (drill 0.4) (layers "F.Cu" "B.Cu") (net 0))
 (via (at 74.1 77.268932) (size 0.8) (drill 0.4) (layers "F.Cu" "B.Cu") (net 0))
 (via (at 74.1 108.65) (size 0.8) (drill 0.4) (layers "F.Cu" "B.Cu") (free) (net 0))
 (via (at 74.1 114.22) (size 0.8) (drill 0.4) (layers "F.Cu" "B.Cu") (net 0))
 (via (at 74.1 84.116664) (size 0.8) (drill 0.4) (layers "F.Cu" "B.Cu") (free) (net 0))
 (via (at 74.1 96.38333) (size 0.8) (drill 0.4) (layers "F.Cu" "B.Cu") (free) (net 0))
 (segment (start 59.2701 96.803216) (end 52.203216 96.803216) (width 0.25) (layer "B.Cu") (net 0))
 (segment (start 74.1 47.316666) (end 74.1 52.654648) (width 0.25) (layer "B.Cu") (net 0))
 (segment (start 74.1 96.38333) (end 74.1 101.883216) (width 0.25) (layer "B.Cu") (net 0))
 (segment (start 59.2701 72.188932) (end 52.161068 72.188932) (width 0.25) (layer "B.Cu") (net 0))
 (segment (start 59.2701 47.574648) (end 52.174648 47.574648) (width 0.25) (layer "B.Cu") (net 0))
 (segment (start 74.1 108.65) (end 74.1 114.22) (width 0.25) (layer "B.Cu") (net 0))
 (segment (start 74.1 71.849998) (end 74.1 77.268932) (width 0.25) (layer "B.Cu") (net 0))
 (segment (start 59.2701 59.88179) (end 52.23179 59.88179) (width 0.25) (layer "B.Cu") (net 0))
 (segment (start 52.23179 59.88179) (end 52.15 59.8) (width 0.25) (layer "B.Cu") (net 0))
 (segment (start 59.2701 121.4175) (end 54.2175 121.4175) (width 0.25) (layer "B.Cu") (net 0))
 (segment (start 52.15 119.35) (end 52.15 37.65) (width 0.25) (layer "B.Cu") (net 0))
 (segment (start 74.1 35.05) (end 74.1 40.347506) (width 0.25) (layer "B.Cu") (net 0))
 (segment (start 52.174648 47.574648) (end 52.15 47.55) (width 0.25) (layer "B.Cu") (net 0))
 (segment (start 74.1 121) (end 74.1 126.4975) (width 0.25) (layer "B.Cu") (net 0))
 (segment (start 59.2701 109.110358) (end 52.189642 109.110358) (width 0.25) (layer "B.Cu") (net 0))
 (segment (start 74.1 59.583332) (end 74.1 64.96179) (width 0.25) (layer "B.Cu") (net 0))
 (segment (start 54.2175 121.4175) (end 52.15 119.35) (width 0.25) (layer "B.Cu") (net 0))
 (segment (start 54.532494 35.267506) (end 59.2701 35.267506) (width 0.25) (layer "B.Cu") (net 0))
 (segment (start 52.189642 109.110358) (end 52.15 109.15) (width 0.25) (layer "B.Cu") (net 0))
 (segment (start 74.1 84.116664) (end 74.1 89.576074) (width 0.25) (layer "B.Cu") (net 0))
 (segment (start 52.15 37.65) (end 54.532494 35.267506) (width 0.25) (layer "B.Cu") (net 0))
 (segment (start 59.2701 84.496074) (end 52.196074 84.496074) (width 0.25) (layer "B.Cu") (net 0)))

